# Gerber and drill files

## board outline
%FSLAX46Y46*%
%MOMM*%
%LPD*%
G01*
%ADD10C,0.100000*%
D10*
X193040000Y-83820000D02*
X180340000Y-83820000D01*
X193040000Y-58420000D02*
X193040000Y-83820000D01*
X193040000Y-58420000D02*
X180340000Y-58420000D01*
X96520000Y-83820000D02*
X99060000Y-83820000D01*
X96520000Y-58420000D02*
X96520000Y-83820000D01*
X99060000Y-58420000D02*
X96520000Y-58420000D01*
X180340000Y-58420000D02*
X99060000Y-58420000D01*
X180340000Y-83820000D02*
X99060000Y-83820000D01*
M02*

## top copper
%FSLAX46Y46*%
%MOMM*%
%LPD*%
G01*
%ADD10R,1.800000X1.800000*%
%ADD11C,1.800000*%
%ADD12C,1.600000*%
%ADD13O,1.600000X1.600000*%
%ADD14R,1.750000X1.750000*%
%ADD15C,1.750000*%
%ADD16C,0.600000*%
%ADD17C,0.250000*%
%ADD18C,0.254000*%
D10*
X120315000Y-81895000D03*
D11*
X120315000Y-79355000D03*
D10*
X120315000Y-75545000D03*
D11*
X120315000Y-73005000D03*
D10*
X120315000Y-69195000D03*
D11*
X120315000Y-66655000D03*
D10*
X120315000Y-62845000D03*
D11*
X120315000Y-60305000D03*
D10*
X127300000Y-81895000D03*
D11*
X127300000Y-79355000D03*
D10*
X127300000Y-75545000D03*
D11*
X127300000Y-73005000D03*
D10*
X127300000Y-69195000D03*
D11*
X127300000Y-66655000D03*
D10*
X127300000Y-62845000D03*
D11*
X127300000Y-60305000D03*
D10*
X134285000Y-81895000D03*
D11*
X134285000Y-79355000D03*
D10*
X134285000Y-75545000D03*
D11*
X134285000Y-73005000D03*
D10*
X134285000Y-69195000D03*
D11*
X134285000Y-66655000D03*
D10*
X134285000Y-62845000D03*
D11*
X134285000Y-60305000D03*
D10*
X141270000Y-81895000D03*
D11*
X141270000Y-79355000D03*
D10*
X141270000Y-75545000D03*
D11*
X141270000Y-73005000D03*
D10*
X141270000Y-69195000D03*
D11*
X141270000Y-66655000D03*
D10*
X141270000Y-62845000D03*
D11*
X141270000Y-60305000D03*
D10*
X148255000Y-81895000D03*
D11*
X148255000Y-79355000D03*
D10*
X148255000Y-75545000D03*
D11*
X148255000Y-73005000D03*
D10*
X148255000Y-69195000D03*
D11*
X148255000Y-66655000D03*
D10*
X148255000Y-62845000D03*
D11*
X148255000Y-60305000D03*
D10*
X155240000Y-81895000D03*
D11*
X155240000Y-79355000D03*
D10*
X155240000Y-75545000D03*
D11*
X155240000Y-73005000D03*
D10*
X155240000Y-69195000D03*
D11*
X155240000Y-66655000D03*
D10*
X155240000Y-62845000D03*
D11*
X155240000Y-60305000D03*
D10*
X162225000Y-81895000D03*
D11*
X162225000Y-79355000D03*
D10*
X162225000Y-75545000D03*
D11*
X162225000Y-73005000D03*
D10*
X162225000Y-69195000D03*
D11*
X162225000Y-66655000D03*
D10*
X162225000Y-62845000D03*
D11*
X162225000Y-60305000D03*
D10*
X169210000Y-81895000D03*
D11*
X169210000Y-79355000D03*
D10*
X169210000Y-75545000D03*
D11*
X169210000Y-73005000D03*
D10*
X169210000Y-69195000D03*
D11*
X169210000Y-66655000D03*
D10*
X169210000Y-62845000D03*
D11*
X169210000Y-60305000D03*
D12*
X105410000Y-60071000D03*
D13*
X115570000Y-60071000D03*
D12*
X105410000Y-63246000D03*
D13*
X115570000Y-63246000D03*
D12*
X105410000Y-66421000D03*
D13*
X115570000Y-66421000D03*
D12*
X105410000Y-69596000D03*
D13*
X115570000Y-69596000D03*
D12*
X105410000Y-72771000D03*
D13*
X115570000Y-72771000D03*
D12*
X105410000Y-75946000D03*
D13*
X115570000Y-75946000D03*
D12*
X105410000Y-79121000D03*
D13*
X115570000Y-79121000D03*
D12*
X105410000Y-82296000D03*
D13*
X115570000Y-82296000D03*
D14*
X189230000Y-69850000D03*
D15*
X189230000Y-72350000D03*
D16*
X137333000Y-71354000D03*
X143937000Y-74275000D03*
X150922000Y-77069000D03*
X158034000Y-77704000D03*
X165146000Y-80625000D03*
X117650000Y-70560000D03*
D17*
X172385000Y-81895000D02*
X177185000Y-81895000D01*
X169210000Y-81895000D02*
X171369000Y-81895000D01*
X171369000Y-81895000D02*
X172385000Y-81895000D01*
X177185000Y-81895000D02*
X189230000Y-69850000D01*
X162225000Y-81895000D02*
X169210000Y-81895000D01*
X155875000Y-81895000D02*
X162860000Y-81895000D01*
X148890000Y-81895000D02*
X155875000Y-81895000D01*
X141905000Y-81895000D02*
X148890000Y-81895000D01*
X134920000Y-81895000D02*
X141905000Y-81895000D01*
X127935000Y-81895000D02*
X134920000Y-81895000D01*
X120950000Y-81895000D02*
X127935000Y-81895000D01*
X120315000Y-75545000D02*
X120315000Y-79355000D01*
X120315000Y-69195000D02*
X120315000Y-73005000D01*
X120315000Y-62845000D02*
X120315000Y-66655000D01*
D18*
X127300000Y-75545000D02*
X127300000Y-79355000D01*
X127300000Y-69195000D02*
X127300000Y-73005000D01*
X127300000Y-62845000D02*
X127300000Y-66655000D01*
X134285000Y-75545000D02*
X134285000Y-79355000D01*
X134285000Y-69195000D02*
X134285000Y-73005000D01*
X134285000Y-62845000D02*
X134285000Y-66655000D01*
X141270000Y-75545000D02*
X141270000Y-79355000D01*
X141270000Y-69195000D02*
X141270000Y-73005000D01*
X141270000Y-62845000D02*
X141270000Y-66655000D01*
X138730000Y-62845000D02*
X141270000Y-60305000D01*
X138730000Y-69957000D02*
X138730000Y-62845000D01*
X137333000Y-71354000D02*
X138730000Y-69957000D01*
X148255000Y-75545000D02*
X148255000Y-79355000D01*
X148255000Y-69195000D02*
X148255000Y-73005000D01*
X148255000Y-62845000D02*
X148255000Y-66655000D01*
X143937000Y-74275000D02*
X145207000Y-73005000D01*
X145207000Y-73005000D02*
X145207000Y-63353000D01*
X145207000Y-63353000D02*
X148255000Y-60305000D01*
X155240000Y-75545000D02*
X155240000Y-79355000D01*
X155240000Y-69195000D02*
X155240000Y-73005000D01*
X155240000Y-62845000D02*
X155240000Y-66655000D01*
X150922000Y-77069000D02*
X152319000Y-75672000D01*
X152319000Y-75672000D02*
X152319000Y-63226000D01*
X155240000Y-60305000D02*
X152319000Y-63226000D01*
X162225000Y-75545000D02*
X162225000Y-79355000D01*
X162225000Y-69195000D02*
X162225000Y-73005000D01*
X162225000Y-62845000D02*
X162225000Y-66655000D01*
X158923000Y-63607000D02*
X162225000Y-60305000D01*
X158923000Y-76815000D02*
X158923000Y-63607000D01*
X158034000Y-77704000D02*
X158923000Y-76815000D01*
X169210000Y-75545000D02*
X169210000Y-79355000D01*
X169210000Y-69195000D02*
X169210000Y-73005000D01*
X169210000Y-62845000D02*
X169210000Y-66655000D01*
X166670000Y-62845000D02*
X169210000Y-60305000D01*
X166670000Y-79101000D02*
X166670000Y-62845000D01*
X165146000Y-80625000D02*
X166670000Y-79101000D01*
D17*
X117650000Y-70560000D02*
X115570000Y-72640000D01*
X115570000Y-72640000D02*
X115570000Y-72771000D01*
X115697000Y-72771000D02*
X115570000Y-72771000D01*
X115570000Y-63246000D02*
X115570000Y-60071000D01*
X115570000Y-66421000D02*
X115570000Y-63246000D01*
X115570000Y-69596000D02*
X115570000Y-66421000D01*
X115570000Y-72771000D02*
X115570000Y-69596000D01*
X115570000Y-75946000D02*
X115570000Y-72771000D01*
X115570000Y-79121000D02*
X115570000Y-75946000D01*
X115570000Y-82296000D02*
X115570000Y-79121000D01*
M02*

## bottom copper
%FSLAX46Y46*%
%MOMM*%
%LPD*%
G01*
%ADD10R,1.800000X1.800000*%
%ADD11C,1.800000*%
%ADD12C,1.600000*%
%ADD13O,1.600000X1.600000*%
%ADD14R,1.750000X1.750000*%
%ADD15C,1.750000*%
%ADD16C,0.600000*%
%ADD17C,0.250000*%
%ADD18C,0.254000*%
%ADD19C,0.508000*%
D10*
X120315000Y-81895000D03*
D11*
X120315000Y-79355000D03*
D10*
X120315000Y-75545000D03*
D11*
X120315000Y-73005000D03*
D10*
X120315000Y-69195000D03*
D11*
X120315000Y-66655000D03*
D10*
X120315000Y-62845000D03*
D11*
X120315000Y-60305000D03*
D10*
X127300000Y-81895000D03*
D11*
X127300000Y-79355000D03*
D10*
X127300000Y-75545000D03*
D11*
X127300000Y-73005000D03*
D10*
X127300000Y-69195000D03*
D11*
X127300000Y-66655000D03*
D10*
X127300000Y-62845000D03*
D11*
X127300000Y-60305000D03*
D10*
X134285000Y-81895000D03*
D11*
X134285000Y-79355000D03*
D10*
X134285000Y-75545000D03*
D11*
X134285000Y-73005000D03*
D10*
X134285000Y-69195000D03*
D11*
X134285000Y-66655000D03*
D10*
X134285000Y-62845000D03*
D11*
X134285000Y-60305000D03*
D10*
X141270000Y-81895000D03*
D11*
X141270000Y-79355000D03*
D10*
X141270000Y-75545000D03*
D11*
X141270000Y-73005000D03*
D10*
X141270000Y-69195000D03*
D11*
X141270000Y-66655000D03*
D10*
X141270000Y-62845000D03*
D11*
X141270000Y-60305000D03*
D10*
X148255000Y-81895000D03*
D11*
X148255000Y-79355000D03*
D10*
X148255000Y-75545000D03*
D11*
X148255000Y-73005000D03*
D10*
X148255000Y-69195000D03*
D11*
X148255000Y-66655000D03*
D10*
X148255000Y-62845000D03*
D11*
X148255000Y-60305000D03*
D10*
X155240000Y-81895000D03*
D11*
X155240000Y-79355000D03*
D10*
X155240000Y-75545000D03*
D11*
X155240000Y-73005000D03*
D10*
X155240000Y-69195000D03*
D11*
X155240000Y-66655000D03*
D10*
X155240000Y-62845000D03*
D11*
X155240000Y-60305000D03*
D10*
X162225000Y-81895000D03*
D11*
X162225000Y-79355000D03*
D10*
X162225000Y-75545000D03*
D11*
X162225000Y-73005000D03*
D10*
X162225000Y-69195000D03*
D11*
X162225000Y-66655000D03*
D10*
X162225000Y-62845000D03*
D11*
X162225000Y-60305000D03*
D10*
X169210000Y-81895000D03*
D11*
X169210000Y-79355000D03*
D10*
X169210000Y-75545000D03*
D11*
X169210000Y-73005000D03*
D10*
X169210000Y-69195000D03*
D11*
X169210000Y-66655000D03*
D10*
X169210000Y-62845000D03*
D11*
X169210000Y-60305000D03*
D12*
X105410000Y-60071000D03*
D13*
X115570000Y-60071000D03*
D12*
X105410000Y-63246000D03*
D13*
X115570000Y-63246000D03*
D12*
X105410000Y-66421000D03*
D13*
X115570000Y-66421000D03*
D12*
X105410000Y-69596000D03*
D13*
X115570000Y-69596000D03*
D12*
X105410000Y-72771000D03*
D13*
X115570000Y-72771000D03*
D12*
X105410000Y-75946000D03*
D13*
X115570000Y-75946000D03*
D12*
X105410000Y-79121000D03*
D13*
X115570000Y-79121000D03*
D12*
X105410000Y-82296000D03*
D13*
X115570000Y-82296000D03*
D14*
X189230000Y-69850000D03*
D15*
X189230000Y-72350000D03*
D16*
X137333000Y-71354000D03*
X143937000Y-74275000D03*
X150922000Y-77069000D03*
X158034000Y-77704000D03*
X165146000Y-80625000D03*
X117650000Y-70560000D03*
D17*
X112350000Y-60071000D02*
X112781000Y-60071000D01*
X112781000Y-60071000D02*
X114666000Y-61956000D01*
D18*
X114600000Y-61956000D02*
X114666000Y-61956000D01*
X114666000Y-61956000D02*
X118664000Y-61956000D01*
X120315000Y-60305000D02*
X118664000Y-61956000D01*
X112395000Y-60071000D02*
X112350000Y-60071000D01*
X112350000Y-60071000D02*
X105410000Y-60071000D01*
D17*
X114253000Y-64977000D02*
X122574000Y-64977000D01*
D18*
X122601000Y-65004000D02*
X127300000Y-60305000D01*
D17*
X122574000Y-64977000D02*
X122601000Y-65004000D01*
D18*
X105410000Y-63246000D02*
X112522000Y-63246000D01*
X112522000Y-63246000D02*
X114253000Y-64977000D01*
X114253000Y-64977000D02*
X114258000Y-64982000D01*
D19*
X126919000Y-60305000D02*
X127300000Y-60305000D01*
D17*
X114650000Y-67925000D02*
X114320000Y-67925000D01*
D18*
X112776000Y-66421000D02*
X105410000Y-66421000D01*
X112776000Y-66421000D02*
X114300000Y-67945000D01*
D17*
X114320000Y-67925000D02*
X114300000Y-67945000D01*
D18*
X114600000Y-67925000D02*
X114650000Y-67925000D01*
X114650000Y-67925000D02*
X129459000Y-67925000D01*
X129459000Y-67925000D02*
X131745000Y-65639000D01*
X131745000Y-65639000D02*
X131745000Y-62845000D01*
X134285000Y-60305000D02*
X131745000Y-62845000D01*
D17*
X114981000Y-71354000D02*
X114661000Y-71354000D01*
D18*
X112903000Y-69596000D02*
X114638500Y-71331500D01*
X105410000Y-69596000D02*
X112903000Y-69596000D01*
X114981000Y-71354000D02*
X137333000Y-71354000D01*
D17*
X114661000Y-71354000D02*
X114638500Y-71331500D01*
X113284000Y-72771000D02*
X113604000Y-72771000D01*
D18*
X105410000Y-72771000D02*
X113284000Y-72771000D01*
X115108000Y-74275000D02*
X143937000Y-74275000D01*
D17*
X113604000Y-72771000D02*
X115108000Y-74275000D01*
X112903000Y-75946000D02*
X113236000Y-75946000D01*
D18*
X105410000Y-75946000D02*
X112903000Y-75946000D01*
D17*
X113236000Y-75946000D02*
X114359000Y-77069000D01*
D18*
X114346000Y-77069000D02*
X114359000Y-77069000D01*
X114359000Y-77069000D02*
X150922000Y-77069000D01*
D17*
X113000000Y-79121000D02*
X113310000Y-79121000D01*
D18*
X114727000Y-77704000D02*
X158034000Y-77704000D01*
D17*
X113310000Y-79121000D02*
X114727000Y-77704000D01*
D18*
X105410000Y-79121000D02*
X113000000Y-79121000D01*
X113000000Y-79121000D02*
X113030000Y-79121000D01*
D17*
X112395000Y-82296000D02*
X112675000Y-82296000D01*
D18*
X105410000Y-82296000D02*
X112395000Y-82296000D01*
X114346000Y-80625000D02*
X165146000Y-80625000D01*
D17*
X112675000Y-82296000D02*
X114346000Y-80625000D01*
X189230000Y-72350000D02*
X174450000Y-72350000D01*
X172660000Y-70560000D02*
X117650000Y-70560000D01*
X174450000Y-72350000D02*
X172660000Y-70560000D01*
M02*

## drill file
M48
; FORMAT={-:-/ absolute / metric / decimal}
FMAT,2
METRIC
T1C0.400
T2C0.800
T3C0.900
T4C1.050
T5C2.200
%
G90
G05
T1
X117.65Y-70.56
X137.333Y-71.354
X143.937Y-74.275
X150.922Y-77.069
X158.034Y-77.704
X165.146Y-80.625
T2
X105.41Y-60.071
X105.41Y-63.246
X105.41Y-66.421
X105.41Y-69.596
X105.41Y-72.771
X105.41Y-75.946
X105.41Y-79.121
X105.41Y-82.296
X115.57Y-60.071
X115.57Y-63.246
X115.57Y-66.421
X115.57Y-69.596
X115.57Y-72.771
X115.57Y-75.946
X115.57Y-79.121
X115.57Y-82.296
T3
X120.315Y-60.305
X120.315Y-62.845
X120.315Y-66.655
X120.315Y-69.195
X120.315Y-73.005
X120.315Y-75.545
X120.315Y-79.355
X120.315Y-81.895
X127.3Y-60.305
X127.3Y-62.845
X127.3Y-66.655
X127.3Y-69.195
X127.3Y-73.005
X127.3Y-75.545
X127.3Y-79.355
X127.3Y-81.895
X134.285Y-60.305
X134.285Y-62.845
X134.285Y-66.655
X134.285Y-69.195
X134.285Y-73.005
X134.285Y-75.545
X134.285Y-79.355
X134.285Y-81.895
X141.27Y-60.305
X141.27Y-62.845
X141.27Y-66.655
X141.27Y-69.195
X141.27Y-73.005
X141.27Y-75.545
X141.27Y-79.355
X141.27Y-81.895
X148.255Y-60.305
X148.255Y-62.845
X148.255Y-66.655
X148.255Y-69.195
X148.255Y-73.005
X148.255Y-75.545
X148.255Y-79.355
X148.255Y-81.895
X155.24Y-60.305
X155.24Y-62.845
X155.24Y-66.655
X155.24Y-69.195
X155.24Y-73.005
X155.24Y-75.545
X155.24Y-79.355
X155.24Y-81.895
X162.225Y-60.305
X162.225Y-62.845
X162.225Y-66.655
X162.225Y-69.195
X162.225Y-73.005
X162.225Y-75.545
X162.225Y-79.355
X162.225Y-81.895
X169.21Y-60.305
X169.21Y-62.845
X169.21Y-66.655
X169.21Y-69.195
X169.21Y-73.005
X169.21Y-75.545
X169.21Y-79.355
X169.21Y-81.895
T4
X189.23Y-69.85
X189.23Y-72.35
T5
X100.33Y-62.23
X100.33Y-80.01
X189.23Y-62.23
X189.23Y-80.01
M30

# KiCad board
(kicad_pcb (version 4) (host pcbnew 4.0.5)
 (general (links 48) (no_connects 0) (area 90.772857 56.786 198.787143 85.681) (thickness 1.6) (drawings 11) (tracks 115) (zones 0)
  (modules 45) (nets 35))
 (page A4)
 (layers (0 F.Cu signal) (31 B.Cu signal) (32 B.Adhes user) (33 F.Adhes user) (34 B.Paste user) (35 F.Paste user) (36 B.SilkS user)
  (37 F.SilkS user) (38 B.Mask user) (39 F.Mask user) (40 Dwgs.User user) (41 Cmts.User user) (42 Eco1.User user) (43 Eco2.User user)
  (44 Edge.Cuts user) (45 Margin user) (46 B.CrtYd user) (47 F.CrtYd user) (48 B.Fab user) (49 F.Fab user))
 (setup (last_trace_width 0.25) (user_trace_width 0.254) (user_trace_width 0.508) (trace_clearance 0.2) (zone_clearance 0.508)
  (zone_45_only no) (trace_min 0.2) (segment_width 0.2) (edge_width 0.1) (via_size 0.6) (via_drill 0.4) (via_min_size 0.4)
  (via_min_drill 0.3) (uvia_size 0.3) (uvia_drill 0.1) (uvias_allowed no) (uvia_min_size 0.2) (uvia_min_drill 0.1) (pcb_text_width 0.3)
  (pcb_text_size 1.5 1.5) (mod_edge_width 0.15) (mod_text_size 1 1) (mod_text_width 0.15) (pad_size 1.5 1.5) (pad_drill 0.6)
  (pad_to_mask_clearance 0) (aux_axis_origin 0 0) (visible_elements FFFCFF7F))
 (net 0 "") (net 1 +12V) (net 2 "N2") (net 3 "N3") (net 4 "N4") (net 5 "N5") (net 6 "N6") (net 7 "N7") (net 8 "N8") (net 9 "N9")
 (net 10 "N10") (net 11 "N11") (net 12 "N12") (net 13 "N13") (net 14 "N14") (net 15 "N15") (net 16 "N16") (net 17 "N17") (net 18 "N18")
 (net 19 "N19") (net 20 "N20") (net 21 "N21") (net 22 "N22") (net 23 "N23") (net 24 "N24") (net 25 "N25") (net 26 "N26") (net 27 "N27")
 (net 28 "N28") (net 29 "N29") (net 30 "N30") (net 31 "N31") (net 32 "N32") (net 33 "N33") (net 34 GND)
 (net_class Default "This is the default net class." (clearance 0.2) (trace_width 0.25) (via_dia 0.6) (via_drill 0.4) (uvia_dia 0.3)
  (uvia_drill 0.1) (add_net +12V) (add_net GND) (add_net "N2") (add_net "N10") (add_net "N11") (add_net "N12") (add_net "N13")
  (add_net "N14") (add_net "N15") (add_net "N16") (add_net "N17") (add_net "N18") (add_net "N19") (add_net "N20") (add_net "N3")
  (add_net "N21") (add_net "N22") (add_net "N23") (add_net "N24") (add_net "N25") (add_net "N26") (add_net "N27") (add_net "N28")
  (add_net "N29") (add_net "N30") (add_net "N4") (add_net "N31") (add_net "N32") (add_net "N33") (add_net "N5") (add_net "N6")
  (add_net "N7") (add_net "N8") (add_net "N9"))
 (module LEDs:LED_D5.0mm (layer F.Cu) (at 120.315 81.895 90)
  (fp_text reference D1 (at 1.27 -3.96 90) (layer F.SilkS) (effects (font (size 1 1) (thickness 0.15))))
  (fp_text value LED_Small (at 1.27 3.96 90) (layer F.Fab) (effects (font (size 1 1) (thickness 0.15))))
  (pad 1 thru_hole rect (at 0 0 90) (size 1.8 1.8) (drill 0.9) (layers *.Cu *.Mask) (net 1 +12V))
  (pad 2 thru_hole circle (at 2.54 0 90) (size 1.8 1.8) (drill 0.9) (layers *.Cu *.Mask) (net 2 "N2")))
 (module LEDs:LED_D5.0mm (layer F.Cu) (at 120.315 75.545 90)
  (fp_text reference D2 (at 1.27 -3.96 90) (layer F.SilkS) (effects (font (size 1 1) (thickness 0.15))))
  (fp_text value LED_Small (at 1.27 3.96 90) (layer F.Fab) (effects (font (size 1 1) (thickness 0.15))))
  (pad 1 thru_hole rect (at 0 0 90) (size 1.8 1.8) (drill 0.9) (layers *.Cu *.Mask) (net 2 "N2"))
  (pad 2 thru_hole circle (at 2.54 0 90) (size 1.8 1.8) (drill 0.9) (layers *.Cu *.Mask) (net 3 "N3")))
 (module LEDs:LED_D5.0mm (layer F.Cu) (at 120.315 69.195 90)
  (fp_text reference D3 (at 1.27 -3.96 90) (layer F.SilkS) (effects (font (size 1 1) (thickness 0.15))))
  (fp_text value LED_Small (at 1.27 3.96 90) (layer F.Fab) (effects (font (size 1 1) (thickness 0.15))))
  (pad 1 thru_hole rect (at 0 0 90) (size 1.8 1.8) (drill 0.9) (layers *.Cu *.Mask) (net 3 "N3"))
  (pad 2 thru_hole circle (at 2.54 0 90) (size 1.8 1.8) (drill 0.9) (layers *.Cu *.Mask) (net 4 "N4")))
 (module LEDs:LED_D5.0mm (layer F.Cu) (at 120.315 62.845 90)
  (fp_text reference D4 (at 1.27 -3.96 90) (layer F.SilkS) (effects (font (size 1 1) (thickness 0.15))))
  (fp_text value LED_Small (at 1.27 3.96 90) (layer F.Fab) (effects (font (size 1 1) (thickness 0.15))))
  (pad 1 thru_hole rect (at 0 0 90) (size 1.8 1.8) (drill 0.9) (layers *.Cu *.Mask) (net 4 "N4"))
  (pad 2 thru_hole circle (at 2.54 0 90) (size 1.8 1.8) (drill 0.9) (layers *.Cu *.Mask) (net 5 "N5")))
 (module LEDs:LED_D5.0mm (layer F.Cu) (at 127.3 81.895 90)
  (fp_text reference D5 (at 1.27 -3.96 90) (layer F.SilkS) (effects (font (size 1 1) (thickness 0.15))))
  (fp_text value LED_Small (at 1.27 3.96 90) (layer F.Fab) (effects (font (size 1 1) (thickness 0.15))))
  (pad 1 thru_hole rect (at 0 0 90) (size 1.8 1.8) (drill 0.9) (layers *.Cu *.Mask) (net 1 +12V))
  (pad 2 thru_hole circle (at 2.54 0 90) (size 1.8 1.8) (drill 0.9) (layers *.Cu *.Mask) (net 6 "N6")))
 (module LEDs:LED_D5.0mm (layer F.Cu) (at 127.3 75.545 90)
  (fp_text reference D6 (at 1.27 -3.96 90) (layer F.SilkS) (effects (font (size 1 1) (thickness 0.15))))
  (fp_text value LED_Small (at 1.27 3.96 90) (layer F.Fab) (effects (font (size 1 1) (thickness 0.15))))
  (pad 1 thru_hole rect (at 0 0 90) (size 1.8 1.8) (drill 0.9) (layers *.Cu *.Mask) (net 6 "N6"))
  (pad 2 thru_hole circle (at 2.54 0 90) (size 1.8 1.8) (drill 0.9) (layers *.Cu *.Mask) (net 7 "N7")))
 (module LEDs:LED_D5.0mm (layer F.Cu) (at 127.3 69.195 90)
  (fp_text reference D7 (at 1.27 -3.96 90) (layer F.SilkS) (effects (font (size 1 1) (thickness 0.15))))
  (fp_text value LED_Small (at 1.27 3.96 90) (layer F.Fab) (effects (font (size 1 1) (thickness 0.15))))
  (pad 1 thru_hole rect (at 0 0 90) (size 1.8 1.8) (drill 0.9) (layers *.Cu *.Mask) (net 7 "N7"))
  (pad 2 thru_hole circle (at 2.54 0 90) (size 1.8 1.8) (drill 0.9) (layers *.Cu *.Mask) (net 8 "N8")))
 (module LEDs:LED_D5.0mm (layer F.Cu) (at 127.3 62.845 90)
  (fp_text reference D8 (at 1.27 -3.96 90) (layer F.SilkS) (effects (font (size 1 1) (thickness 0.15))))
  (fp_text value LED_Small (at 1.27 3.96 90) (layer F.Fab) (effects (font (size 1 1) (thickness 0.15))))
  (pad 1 thru_hole rect (at 0 0 90) (size 1.8 1.8) (drill 0.9) (layers *.Cu *.Mask) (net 8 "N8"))
  (pad 2 thru_hole circle (at 2.54 0 90) (size 1.8 1.8) (drill 0.9) (layers *.Cu *.Mask) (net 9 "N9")))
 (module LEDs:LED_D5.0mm (layer F.Cu) (at 134.285 81.895 90)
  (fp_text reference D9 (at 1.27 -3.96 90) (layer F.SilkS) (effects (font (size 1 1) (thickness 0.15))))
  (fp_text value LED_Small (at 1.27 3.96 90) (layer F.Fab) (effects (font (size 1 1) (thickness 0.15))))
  (pad 1 thru_hole rect (at 0 0 90) (size 1.8 1.8) (drill 0.9) (layers *.Cu *.Mask) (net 1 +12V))
  (pad 2 thru_hole circle (at 2.54 0 90) (size 1.8 1.8) (drill 0.9) (layers *.Cu *.Mask) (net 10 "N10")))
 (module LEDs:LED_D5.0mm (layer F.Cu) (at 134.285 75.545 90)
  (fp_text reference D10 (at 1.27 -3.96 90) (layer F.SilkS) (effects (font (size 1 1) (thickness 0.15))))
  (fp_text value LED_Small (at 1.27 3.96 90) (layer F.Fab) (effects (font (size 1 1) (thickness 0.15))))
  (pad 1 thru_hole rect (at 0 0 90) (size 1.8 1.8) (drill 0.9) (layers *.Cu *.Mask) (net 10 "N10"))
  (pad 2 thru_hole circle (at 2.54 0 90) (size 1.8 1.8) (drill 0.9) (layers *.Cu *.Mask) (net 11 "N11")))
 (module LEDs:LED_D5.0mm (layer F.Cu) (at 134.285 69.195 90)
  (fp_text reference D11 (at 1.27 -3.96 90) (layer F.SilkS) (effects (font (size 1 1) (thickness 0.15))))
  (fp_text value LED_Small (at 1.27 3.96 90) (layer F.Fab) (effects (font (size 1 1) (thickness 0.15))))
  (pad 1 thru_hole rect (at 0 0 90) (size 1.8 1.8) (drill 0.9) (layers *.Cu *.Mask) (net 11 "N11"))
  (pad 2 thru_hole circle (at 2.54 0 90) (size 1.8 1.8) (drill 0.9) (layers *.Cu *.Mask) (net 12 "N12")))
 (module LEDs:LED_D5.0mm (layer F.Cu) (at 134.285 62.845 90)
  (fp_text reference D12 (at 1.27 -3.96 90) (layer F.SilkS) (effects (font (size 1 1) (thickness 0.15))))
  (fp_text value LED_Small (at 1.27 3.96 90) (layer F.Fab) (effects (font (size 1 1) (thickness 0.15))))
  (pad 1 thru_hole rect (at 0 0 90) (size 1.8 1.8) (drill 0.9) (layers *.Cu *.Mask) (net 12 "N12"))
  (pad 2 thru_hole circle (at 2.54 0 90) (size 1.8 1.8) (drill 0.9) (layers *.Cu *.Mask) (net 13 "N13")))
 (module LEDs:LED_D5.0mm (layer F.Cu) (at 141.27 81.895 90)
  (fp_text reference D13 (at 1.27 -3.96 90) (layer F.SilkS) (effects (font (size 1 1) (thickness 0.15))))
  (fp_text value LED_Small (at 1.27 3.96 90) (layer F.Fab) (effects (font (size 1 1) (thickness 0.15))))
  (pad 1 thru_hole rect (at 0 0 90) (size 1.8 1.8) (drill 0.9) (layers *.Cu *.Mask) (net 1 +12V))
  (pad 2 thru_hole circle (at 2.54 0 90) (size 1.8 1.8) (drill 0.9) (layers *.Cu *.Mask) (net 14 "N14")))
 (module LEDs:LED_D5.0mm (layer F.Cu) (at 141.27 75.545 90)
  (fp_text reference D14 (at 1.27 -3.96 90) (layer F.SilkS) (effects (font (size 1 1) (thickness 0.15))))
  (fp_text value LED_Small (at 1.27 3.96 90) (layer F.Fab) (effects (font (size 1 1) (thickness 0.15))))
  (pad 1 thru_hole rect (at 0 0 90) (size 1.8 1.8) (drill 0.9) (layers *.Cu *.Mask) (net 14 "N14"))
  (pad 2 thru_hole circle (at 2.54 0 90) (size 1.8 1.8) (drill 0.9) (layers *.Cu *.Mask) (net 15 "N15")))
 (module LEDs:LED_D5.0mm (layer F.Cu) (at 141.27 69.195 90)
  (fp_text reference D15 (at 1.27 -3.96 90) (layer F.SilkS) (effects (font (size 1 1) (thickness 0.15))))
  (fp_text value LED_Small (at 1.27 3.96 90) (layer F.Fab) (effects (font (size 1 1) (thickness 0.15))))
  (pad 1 thru_hole rect (at 0 0 90) (size 1.8 1.8) (drill 0.9) (layers *.Cu *.Mask) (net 15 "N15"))
  (pad 2 thru_hole circle (at 2.54 0 90) (size 1.8 1.8) (drill 0.9) (layers *.Cu *.Mask) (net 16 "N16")))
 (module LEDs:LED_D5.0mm (layer F.Cu) (at 141.27 62.845 90)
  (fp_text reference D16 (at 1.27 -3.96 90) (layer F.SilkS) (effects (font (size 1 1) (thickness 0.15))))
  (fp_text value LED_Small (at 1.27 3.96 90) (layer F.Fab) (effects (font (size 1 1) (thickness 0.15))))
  (pad 1 thru_hole rect (at 0 0 90) (size 1.8 1.8) (drill 0.9) (layers *.Cu *.Mask) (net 16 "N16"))
  (pad 2 thru_hole circle (at 2.54 0 90) (size 1.8 1.8) (drill 0.9) (layers *.Cu *.Mask) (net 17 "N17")))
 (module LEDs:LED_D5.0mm (layer F.Cu) (at 148.255 81.895 90)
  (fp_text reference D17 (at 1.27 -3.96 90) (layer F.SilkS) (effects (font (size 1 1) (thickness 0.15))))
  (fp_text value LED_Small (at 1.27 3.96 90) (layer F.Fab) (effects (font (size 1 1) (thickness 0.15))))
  (pad 1 thru_hole rect (at 0 0 90) (size 1.8 1.8) (drill 0.9) (layers *.Cu *.Mask) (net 1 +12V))
  (pad 2 thru_hole circle (at 2.54 0 90) (size 1.8 1.8) (drill 0.9) (layers *.Cu *.Mask) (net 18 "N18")))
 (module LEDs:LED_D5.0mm (layer F.Cu) (at 148.255 75.545 90)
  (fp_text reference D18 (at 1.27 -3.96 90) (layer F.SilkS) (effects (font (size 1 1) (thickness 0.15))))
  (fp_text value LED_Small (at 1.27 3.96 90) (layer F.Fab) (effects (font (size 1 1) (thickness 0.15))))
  (pad 1 thru_hole rect (at 0 0 90) (size 1.8 1.8) (drill 0.9) (layers *.Cu *.Mask) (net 18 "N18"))
  (pad 2 thru_hole circle (at 2.54 0 90) (size 1.8 1.8) (drill 0.9) (layers *.Cu *.Mask) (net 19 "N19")))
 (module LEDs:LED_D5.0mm (layer F.Cu) (at 148.255 69.195 90)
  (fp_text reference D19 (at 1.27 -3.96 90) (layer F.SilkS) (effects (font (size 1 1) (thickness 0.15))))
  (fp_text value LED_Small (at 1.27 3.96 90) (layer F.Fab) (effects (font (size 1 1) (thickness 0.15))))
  (pad 1 thru_hole rect (at 0 0 90) (size 1.8 1.8) (drill 0.9) (layers *.Cu *.Mask) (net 19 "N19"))
  (pad 2 thru_hole circle (at 2.54 0 90) (size 1.8 1.8) (drill 0.9) (layers *.Cu *.Mask) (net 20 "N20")))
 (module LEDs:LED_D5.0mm (layer F.Cu) (at 148.255 62.845 90)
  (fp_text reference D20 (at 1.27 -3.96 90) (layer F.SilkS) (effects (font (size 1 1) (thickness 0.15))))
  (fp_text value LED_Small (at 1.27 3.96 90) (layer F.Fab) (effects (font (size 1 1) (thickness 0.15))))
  (pad 1 thru_hole rect (at 0 0 90) (size 1.8 1.8) (drill 0.9) (layers *.Cu *.Mask) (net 20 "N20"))
  (pad 2 thru_hole circle (at 2.54 0 90) (size 1.8 1.8) (drill 0.9) (layers *.Cu *.Mask) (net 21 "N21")))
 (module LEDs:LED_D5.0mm (layer F.Cu) (at 155.24 81.895 90)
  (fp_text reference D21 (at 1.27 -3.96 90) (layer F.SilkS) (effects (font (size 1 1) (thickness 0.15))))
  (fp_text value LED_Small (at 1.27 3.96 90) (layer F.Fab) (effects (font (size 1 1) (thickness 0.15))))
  (pad 1 thru_hole rect (at 0 0 90) (size 1.8 1.8) (drill 0.9) (layers *.Cu *.Mask) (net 1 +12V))
  (pad 2 thru_hole circle (at 2.54 0 90) (size 1.8 1.8) (drill 0.9) (layers *.Cu *.Mask) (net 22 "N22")))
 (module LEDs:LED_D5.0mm (layer F.Cu) (at 155.24 75.545 90)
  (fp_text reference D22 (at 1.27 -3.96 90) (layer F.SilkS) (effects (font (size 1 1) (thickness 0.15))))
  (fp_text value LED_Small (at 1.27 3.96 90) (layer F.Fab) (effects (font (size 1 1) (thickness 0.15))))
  (pad 1 thru_hole rect (at 0 0 90) (size 1.8 1.8) (drill 0.9) (layers *.Cu *.Mask) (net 22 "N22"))
  (pad 2 thru_hole circle (at 2.54 0 90) (size 1.8 1.8) (drill 0.9) (layers *.Cu *.Mask) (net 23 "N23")))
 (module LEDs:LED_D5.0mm (layer F.Cu) (at 155.24 69.195 90)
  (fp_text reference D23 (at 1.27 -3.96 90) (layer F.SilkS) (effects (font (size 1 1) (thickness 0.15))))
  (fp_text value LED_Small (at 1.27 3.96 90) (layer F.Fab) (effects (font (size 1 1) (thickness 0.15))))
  (pad 1 thru_hole rect (at 0 0 90) (size 1.8 1.8) (drill 0.9) (layers *.Cu *.Mask) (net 23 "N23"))
  (pad 2 thru_hole circle (at 2.54 0 90) (size 1.8 1.8) (drill 0.9) (layers *.Cu *.Mask) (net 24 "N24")))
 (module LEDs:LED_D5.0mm (layer F.Cu) (at 155.24 62.845 90)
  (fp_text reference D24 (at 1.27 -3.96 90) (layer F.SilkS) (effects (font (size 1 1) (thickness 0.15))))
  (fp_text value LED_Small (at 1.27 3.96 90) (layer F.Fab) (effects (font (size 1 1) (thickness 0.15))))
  (pad 1 thru_hole rect (at 0 0 90) (size 1.8 1.8) (drill 0.9) (layers *.Cu *.Mask) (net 24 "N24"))
  (pad 2 thru_hole circle (at 2.54 0 90) (size 1.8 1.8) (drill 0.9) (layers *.Cu *.Mask) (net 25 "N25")))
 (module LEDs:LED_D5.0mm (layer F.Cu) (at 162.225 81.895 90)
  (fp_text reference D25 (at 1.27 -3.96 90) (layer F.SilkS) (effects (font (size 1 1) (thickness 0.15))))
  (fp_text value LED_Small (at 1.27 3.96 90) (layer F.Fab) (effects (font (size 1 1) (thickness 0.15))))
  (pad 1 thru_hole rect (at 0 0 90) (size 1.8 1.8) (drill 0.9) (layers *.Cu *.Mask) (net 1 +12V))
  (pad 2 thru_hole circle (at 2.54 0 90) (size 1.8 1.8) (drill 0.9) (layers *.Cu *.Mask) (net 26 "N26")))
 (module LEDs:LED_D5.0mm (layer F.Cu) (at 162.225 75.545 90)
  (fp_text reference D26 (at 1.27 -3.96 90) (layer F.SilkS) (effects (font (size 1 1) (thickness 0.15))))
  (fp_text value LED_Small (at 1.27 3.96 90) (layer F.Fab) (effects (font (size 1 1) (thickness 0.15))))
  (pad 1 thru_hole rect (at 0 0 90) (size 1.8 1.8) (drill 0.9) (layers *.Cu *.Mask) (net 26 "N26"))
  (pad 2 thru_hole circle (at 2.54 0 90) (size 1.8 1.8) (drill 0.9) (layers *.Cu *.Mask) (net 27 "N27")))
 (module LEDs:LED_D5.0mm (layer F.Cu) (at 162.225 69.195 90)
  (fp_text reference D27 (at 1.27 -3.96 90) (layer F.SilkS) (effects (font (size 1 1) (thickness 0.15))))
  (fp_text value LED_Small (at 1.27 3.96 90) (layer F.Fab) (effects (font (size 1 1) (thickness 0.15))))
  (pad 1 thru_hole rect (at 0 0 90) (size 1.8 1.8) (drill 0.9) (layers *.Cu *.Mask) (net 27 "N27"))
  (pad 2 thru_hole circle (at 2.54 0 90) (size 1.8 1.8) (drill 0.9) (layers *.Cu *.Mask) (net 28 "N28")))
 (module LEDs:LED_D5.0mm (layer F.Cu) (at 162.225 62.845 90)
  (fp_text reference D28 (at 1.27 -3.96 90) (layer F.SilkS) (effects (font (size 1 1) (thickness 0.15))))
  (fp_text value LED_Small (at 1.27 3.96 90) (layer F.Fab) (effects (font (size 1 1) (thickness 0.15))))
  (pad 1 thru_hole rect (at 0 0 90) (size 1.8 1.8) (drill 0.9) (layers *.Cu *.Mask) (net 28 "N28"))
  (pad 2 thru_hole circle (at 2.54 0 90) (size 1.8 1.8) (drill 0.9) (layers *.Cu *.Mask) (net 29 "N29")))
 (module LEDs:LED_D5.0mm (layer F.Cu) (at 169.21 81.895 90)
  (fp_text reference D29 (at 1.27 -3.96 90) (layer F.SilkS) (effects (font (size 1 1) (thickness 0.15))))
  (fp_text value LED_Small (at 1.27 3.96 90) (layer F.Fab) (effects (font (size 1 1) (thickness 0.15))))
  (pad 1 thru_hole rect (at 0 0 90) (size 1.8 1.8) (drill 0.9) (layers *.Cu *.Mask) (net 1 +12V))
  (pad 2 thru_hole circle (at 2.54 0 90) (size 1.8 1.8) (drill 0.9) (layers *.Cu *.Mask) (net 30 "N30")))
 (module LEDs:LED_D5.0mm (layer F.Cu) (at 169.21 75.545 90)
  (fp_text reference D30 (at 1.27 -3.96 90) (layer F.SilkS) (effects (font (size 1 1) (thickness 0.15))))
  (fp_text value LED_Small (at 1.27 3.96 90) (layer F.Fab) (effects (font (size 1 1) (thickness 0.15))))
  (pad 1 thru_hole rect (at 0 0 90) (size 1.8 1.8) (drill 0.9) (layers *.Cu *.Mask) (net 30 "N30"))
  (pad 2 thru_hole circle (at 2.54 0 90) (size 1.8 1.8) (drill 0.9) (layers *.Cu *.Mask) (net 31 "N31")))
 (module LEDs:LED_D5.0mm (layer F.Cu) (at 169.21 69.195 90)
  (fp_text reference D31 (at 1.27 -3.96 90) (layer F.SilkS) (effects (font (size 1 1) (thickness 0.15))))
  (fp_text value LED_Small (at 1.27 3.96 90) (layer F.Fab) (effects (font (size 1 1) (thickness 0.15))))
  (pad 1 thru_hole rect (at 0 0 90) (size 1.8 1.8) (drill 0.9) (layers *.Cu *.Mask) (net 31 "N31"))
  (pad 2 thru_hole circle (at 2.54 0 90) (size 1.8 1.8) (drill 0.9) (layers *.Cu *.Mask) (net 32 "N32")))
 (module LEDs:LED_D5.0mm (layer F.Cu) (at 169.21 62.845 90)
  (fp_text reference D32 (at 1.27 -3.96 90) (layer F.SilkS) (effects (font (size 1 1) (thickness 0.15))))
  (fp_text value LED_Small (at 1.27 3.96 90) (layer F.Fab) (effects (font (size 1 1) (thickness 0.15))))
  (pad 1 thru_hole rect (at 0 0 90) (size 1.8 1.8) (drill 0.9) (layers *.Cu *.Mask) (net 32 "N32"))
  (pad 2 thru_hole circle (at 2.54 0 90) (size 1.8 1.8) (drill 0.9) (layers *.Cu *.Mask) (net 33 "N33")))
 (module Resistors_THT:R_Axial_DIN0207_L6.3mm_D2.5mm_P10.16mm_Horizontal (layer F.Cu) (at 105.41 60.071)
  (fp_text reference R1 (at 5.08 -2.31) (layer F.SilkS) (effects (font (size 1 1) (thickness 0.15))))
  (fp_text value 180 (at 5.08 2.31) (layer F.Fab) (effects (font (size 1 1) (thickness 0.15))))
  (pad 1 thru_hole circle (at 0 0) (size 1.6 1.6) (drill 0.8) (layers *.Cu *.Mask) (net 5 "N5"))
  (pad 2 thru_hole oval (at 10.16 0) (size 1.6 1.6) (drill 0.8) (layers *.Cu *.Mask) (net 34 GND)))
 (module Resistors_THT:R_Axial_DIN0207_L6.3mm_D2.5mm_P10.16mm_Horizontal (layer F.Cu) (at 105.41 63.246)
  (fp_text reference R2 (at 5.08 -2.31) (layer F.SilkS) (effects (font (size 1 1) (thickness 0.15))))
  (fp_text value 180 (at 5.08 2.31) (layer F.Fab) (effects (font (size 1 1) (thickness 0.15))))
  (pad 1 thru_hole circle (at 0 0) (size 1.6 1.6) (drill 0.8) (layers *.Cu *.Mask) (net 9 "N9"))
  (pad 2 thru_hole oval (at 10.16 0) (size 1.6 1.6) (drill 0.8) (layers *.Cu *.Mask) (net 34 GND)))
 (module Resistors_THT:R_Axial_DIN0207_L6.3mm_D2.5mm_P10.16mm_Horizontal (layer F.Cu) (at 105.41 66.421)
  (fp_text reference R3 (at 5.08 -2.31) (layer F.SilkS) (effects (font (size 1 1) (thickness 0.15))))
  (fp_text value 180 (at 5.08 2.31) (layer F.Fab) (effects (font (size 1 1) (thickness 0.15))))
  (pad 1 thru_hole circle (at 0 0) (size 1.6 1.6) (drill 0.8) (layers *.Cu *.Mask) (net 13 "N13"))
  (pad 2 thru_hole oval (at 10.16 0) (size 1.6 1.6) (drill 0.8) (layers *.Cu *.Mask) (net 34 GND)))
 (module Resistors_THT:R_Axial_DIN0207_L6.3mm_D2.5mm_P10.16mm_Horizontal (layer F.Cu) (at 105.41 69.596)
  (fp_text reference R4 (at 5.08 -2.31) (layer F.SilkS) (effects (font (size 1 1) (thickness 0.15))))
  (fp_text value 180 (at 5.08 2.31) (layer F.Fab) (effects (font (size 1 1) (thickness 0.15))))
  (pad 1 thru_hole circle (at 0 0) (size 1.6 1.6) (drill 0.8) (layers *.Cu *.Mask) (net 17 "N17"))
  (pad 2 thru_hole oval (at 10.16 0) (size 1.6 1.6) (drill 0.8) (layers *.Cu *.Mask) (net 34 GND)))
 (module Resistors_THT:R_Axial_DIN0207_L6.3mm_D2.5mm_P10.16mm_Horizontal (layer F.Cu) (at 105.41 72.771)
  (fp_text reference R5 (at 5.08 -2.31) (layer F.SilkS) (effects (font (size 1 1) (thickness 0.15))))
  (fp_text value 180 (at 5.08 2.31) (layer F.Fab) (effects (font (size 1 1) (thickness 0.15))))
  (pad 1 thru_hole circle (at 0 0) (size 1.6 1.6) (drill 0.8) (layers *.Cu *.Mask) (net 21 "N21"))
  (pad 2 thru_hole oval (at 10.16 0) (size 1.6 1.6) (drill 0.8) (layers *.Cu *.Mask) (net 34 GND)))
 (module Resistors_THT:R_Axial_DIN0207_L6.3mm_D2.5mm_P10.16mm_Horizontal (layer F.Cu) (at 105.41 75.946)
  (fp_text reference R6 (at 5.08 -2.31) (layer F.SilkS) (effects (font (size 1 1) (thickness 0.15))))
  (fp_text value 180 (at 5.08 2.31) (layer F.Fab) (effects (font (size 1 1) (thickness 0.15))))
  (pad 1 thru_hole circle (at 0 0) (size 1.6 1.6) (drill 0.8) (layers *.Cu *.Mask) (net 25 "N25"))
  (pad 2 thru_hole oval (at 10.16 0) (size 1.6 1.6) (drill 0.8) (layers *.Cu *.Mask) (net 34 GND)))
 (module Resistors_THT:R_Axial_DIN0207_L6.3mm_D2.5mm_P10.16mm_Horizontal (layer F.Cu) (at 105.41 79.121)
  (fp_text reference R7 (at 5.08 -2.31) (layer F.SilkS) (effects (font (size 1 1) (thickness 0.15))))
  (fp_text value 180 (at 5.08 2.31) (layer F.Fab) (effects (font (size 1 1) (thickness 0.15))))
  (pad 1 thru_hole circle (at 0 0) (size 1.6 1.6) (drill 0.8) (layers *.Cu *.Mask) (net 29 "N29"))
  (pad 2 thru_hole oval (at 10.16 0) (size 1.6 1.6) (drill 0.8) (layers *.Cu *.Mask) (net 34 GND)))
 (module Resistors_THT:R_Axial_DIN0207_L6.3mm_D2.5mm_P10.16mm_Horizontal (layer F.Cu) (at 105.41 82.296)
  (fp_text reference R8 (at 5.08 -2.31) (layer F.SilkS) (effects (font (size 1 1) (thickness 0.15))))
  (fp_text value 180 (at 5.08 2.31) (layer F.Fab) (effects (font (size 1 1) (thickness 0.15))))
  (pad 1 thru_hole circle (at 0 0) (size 1.6 1.6) (drill 0.8) (layers *.Cu *.Mask) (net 33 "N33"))
  (pad 2 thru_hole oval (at 10.16 0) (size 1.6 1.6) (drill 0.8) (layers *.Cu *.Mask) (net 34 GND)))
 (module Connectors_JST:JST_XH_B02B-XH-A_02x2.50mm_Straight (layer F.Cu) (at 189.23 69.85 270)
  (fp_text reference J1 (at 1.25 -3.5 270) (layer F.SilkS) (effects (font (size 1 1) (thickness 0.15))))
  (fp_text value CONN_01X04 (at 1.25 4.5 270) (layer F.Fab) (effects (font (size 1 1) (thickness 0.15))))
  (pad 1 thru_hole rect (at 0 0 270) (size 1.75 1.75) (drill 1.05) (layers *.Cu *.Mask) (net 1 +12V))
  (pad 2 thru_hole circle (at 2.5 0 270) (size 1.75 1.75) (drill 1.05) (layers *.Cu *.Mask) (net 34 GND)))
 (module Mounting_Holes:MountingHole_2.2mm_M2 (layer F.Cu) (at 189.23 62.23)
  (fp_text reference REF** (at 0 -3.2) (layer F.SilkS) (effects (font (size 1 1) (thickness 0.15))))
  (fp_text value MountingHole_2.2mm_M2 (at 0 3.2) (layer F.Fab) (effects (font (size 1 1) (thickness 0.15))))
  (pad 1 np_thru_hole circle (at 0 0) (size 2.2 2.2) (drill 2.2) (layers *.Cu *.Mask)))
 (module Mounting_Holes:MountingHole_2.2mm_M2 (layer F.Cu) (at 189.23 80.01)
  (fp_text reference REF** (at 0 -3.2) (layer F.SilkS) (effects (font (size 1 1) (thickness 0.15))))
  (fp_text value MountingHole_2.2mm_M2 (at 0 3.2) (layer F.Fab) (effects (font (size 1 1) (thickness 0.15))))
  (pad 1 np_thru_hole circle (at 0 0) (size 2.2 2.2) (drill 2.2) (layers *.Cu *.Mask)))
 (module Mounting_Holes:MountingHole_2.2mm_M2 (layer F.Cu) (at 100.33 62.23)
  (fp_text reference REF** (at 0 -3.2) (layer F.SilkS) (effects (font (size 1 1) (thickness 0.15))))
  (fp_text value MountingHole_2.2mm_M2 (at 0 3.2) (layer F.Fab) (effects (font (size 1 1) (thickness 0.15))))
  (pad 1 np_thru_hole circle (at 0 0) (size 2.2 2.2) (drill 2.2) (layers *.Cu *.Mask)))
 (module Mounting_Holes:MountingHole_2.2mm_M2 (layer F.Cu) (at 100.33 80.01)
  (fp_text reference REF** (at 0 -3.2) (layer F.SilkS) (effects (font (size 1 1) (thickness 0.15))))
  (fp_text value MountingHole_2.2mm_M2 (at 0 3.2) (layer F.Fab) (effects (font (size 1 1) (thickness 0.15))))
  (pad 1 np_thru_hole circle (at 0 0) (size 2.2 2.2) (drill 2.2) (layers *.Cu *.Mask)))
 (gr_line (start 193.04 83.82) (end 180.34 83.82) (angle 90) (layer Edge.Cuts) (width 0.1))
 (gr_line (start 193.04 58.42) (end 193.04 83.82) (angle 90) (layer Edge.Cuts) (width 0.1))
 (gr_line (start 193.04 58.42) (end 180.34 58.42) (angle 90) (layer Edge.Cuts) (width 0.1))
 (gr_line (start 96.52 83.82) (end 99.06 83.82) (angle 90) (layer Edge.Cuts) (width 0.1))
 (gr_line (start 96.52 58.42) (end 96.52 83.82) (angle 90) (layer Edge.Cuts) (width 0.1))
 (gr_line (start 99.06 58.42) (end 96.52 58.42) (angle 90) (layer Edge.Cuts) (width 0.1))
 (gr_line (start 180.34 58.42) (end 99.06 58.42) (angle 90) (layer Edge.Cuts) (width 0.1))
 (gr_line (start 180.34 83.82) (end 99.06 83.82) (angle 90) (layer Edge.Cuts) (width 0.1))
 (segment (start 172.385 81.895) (end 177.185 81.895) (width 0.25) (layer F.Cu) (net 1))
 (segment (start 169.21 81.895) (end 171.369 81.895) (width 0.25) (layer F.Cu) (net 1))
 (segment (start 171.369 81.895) (end 172.385 81.895) (width 0.25) (layer F.Cu) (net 1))
 (segment (start 177.185 81.895) (end 189.23 69.85) (width 0.25) (layer F.Cu) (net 1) (status 800000))
 (segment (start 162.225 81.895) (end 169.21 81.895) (width 0.25) (layer F.Cu) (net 1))
 (segment (start 155.875 81.895) (end 162.86 81.895) (width 0.25) (layer F.Cu) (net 1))
 (segment (start 148.89 81.895) (end 155.875 81.895) (width 0.25) (layer F.Cu) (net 1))
 (segment (start 141.905 81.895) (end 148.89 81.895) (width 0.25) (layer F.Cu) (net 1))
 (segment (start 134.92 81.895) (end 141.905 81.895) (width 0.25) (layer F.Cu) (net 1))
 (segment (start 127.935 81.895) (end 134.92 81.895) (width 0.25) (layer F.Cu) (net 1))
 (segment (start 120.95 81.895) (end 127.935 81.895) (width 0.25) (layer F.Cu) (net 1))
 (segment (start 120.315 75.545) (end 120.315 79.355) (width 0.25) (layer F.Cu) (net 2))
 (segment (start 120.315 69.195) (end 120.315 73.005) (width 0.25) (layer F.Cu) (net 3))
 (segment (start 120.315 62.845) (end 120.315 66.655) (width 0.25) (layer F.Cu) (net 4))
 (segment (start 112.35 60.071) (end 112.781 60.071) (width 0.25) (layer B.Cu) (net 5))
 (segment (start 112.781 60.071) (end 114.666 61.956) (width 0.25) (layer B.Cu) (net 5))
 (segment (start 114.6 61.956) (end 114.666 61.956) (width 0.254) (layer B.Cu) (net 5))
 (segment (start 114.666 61.956) (end 118.664 61.956) (width 0.254) (layer B.Cu) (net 5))
 (segment (start 120.315 60.305) (end 118.664 61.956) (width 0.254) (layer B.Cu) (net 5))
 (segment (start 112.395 60.071) (end 112.35 60.071) (width 0.254) (layer B.Cu) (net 5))
 (segment (start 112.35 60.071) (end 105.41 60.071) (width 0.254) (layer B.Cu) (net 5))
 (segment (start 127.3 75.545) (end 127.3 79.355) (width 0.254) (layer F.Cu) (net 6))
 (segment (start 127.3 69.195) (end 127.3 73.005) (width 0.254) (layer F.Cu) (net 7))
 (segment (start 127.3 62.845) (end 127.3 66.655) (width 0.254) (layer F.Cu) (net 8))
 (segment (start 114.253 64.977) (end 122.574 64.977) (width 0.25) (layer B.Cu) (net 9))
 (segment (start 122.601 65.004) (end 127.3 60.305) (width 0.254) (layer B.Cu) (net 9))
 (segment (start 122.574 64.977) (end 122.601 65.004) (width 0.25) (layer B.Cu) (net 9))
 (segment (start 105.41 63.246) (end 112.522 63.246) (width 0.254) (layer B.Cu) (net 9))
 (segment (start 112.522 63.246) (end 114.253 64.977) (width 0.254) (layer B.Cu) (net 9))
 (segment (start 114.253 64.977) (end 114.258 64.982) (width 0.254) (layer B.Cu) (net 9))
 (segment (start 126.919 60.305) (end 127.3 60.305) (width 0.508) (layer B.Cu) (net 9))
 (segment (start 134.285 75.545) (end 134.285 79.355) (width 0.254) (layer F.Cu) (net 10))
 (segment (start 134.285 69.195) (end 134.285 73.005) (width 0.254) (layer F.Cu) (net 11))
 (segment (start 134.285 62.845) (end 134.285 66.655) (width 0.254) (layer F.Cu) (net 12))
 (segment (start 114.65 67.925) (end 114.32 67.925) (width 0.25) (layer B.Cu) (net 13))
 (segment (start 112.776 66.421) (end 105.41 66.421) (width 0.254) (layer B.Cu) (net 13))
 (segment (start 112.776 66.421) (end 114.3 67.945) (width 0.254) (layer B.Cu) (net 13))
 (segment (start 114.32 67.925) (end 114.3 67.945) (width 0.25) (layer B.Cu) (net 13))
 (segment (start 114.6 67.925) (end 114.65 67.925) (width 0.254) (layer B.Cu) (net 13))
 (segment (start 114.65 67.925) (end 129.459 67.925) (width 0.254) (layer B.Cu) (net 13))
 (segment (start 129.459 67.925) (end 131.745 65.639) (width 0.254) (layer B.Cu) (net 13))
 (segment (start 131.745 65.639) (end 131.745 62.845) (width 0.254) (layer B.Cu) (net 13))
 (segment (start 134.285 60.305) (end 131.745 62.845) (width 0.254) (layer B.Cu) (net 13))
 (segment (start 141.27 75.545) (end 141.27 79.355) (width 0.254) (layer F.Cu) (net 14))
 (segment (start 141.27 69.195) (end 141.27 73.005) (width 0.254) (layer F.Cu) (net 15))
 (segment (start 141.27 62.845) (end 141.27 66.655) (width 0.254) (layer F.Cu) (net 16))
 (segment (start 114.981 71.354) (end 114.661 71.354) (width 0.25) (layer B.Cu) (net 17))
 (segment (start 112.903 69.596) (end 114.6385 71.3315) (width 0.254) (layer B.Cu) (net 17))
 (segment (start 105.41 69.596) (end 112.903 69.596) (width 0.254) (layer B.Cu) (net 17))
 (segment (start 138.73 62.845) (end 141.27 60.305) (width 0.254) (layer F.Cu) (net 17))
 (segment (start 138.73 69.957) (end 138.73 62.845) (width 0.254) (layer F.Cu) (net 17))
 (segment (start 137.333 71.354) (end 138.73 69.957) (width 0.254) (layer F.Cu) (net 17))
 (via (at 137.333 71.354) (size 0.6) (drill 0.4) (layers F.Cu B.Cu) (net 17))
 (segment (start 114.981 71.354) (end 137.333 71.354) (width 0.254) (layer B.Cu) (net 17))
 (segment (start 114.661 71.354) (end 114.6385 71.3315) (width 0.25) (layer B.Cu) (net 17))
 (segment (start 148.255 75.545) (end 148.255 79.355) (width 0.254) (layer F.Cu) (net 18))
 (segment (start 148.255 69.195) (end 148.255 73.005) (width 0.254) (layer F.Cu) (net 19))
 (segment (start 148.255 62.845) (end 148.255 66.655) (width 0.254) (layer F.Cu) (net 20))
 (segment (start 113.284 72.771) (end 113.604 72.771) (width 0.25) (layer B.Cu) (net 21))
 (segment (start 105.41 72.771) (end 113.284 72.771) (width 0.254) (layer B.Cu) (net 21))
 (segment (start 115.108 74.275) (end 143.937 74.275) (width 0.254) (layer B.Cu) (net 21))
 (via (at 143.937 74.275) (size 0.6) (drill 0.4) (layers F.Cu B.Cu) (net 21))
 (segment (start 143.937 74.275) (end 145.207 73.005) (width 0.254) (layer F.Cu) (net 21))
 (segment (start 145.207 73.005) (end 145.207 63.353) (width 0.254) (layer F.Cu) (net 21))
 (segment (start 145.207 63.353) (end 148.255 60.305) (width 0.254) (layer F.Cu) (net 21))
 (segment (start 113.604 72.771) (end 115.108 74.275) (width 0.25) (layer B.Cu) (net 21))
 (segment (start 155.24 75.545) (end 155.24 79.355) (width 0.254) (layer F.Cu) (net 22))
 (segment (start 155.24 69.195) (end 155.24 73.005) (width 0.254) (layer F.Cu) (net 23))
 (segment (start 155.24 62.845) (end 155.24 66.655) (width 0.254) (layer F.Cu) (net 24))
 (segment (start 112.903 75.946) (end 113.236 75.946) (width 0.25) (layer B.Cu) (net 25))
 (segment (start 105.41 75.946) (end 112.903 75.946) (width 0.254) (layer B.Cu) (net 25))
 (segment (start 113.236 75.946) (end 114.359 77.069) (width 0.25) (layer B.Cu) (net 25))
 (segment (start 114.346 77.069) (end 114.359 77.069) (width 0.254) (layer B.Cu) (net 25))
 (segment (start 114.359 77.069) (end 150.922 77.069) (width 0.254) (layer B.Cu) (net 25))
 (via (at 150.922 77.069) (size 0.6) (drill 0.4) (layers F.Cu B.Cu) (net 25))
 (segment (start 150.922 77.069) (end 152.319 75.672) (width 0.254) (layer F.Cu) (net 25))
 (segment (start 152.319 75.672) (end 152.319 63.226) (width 0.254) (layer F.Cu) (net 25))
 (segment (start 155.24 60.305) (end 152.319 63.226) (width 0.254) (layer F.Cu) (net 25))
 (segment (start 162.225 75.545) (end 162.225 79.355) (width 0.254) (layer F.Cu) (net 26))
 (segment (start 162.225 69.195) (end 162.225 73.005) (width 0.254) (layer F.Cu) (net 27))
 (segment (start 162.225 62.845) (end 162.225 66.655) (width 0.254) (layer F.Cu) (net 28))
 (segment (start 113 79.121) (end 113.31 79.121) (width 0.25) (layer B.Cu) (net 29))
 (segment (start 158.923 63.607) (end 162.225 60.305) (width 0.254) (layer F.Cu) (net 29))
 (segment (start 158.923 76.815) (end 158.923 63.607) (width 0.254) (layer F.Cu) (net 29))
 (segment (start 158.034 77.704) (end 158.923 76.815) (width 0.254) (layer F.Cu) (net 29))
 (via (at 158.034 77.704) (size 0.6) (drill 0.4) (layers F.Cu B.Cu) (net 29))
 (segment (start 114.727 77.704) (end 158.034 77.704) (width 0.254) (layer B.Cu) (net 29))
 (segment (start 113.31 79.121) (end 114.727 77.704) (width 0.25) (layer B.Cu) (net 29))
 (segment (start 105.41 79.121) (end 113 79.121) (width 0.254) (layer B.Cu) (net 29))
 (segment (start 113 79.121) (end 113.03 79.121) (width 0.254) (layer B.Cu) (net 29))
 (segment (start 169.21 75.545) (end 169.21 79.355) (width 0.254) (layer F.Cu) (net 30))
 (segment (start 169.21 69.195) (end 169.21 73.005) (width 0.254) (layer F.Cu) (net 31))
 (segment (start 169.21 62.845) (end 169.21 66.655) (width 0.254) (layer F.Cu) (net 32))
 (segment (start 112.395 82.296) (end 112.675 82.296) (width 0.25) (layer B.Cu) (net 33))
 (segment (start 105.41 82.296) (end 112.395 82.296) (width 0.254) (layer B.Cu) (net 33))
 (segment (start 166.67 62.845) (end 169.21 60.305) (width 0.254) (layer F.Cu) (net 33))
 (segment (start 166.67 79.101) (end 166.67 62.845) (width 0.254) (layer F.Cu) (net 33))
 (segment (start 165.146 80.625) (end 166.67 79.101) (width 0.254) (layer F.Cu) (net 33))
 (via (at 165.146 80.625) (size 0.6) (drill 0.4) (layers F.Cu B.Cu) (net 33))
 (segment (start 114.346 80.625) (end 165.146 80.625) (width 0.254) (layer B.Cu) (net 33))
 (segment (start 112.675 82.296) (end 114.346 80.625) (width 0.25) (layer B.Cu) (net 33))
 (segment (start 189.23 72.35) (end 174.45 72.35) (width 0.25) (layer B.Cu) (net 34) (status 400000))
 (segment (start 117.65 70.56) (end 115.57 72.64) (width 0.25) (layer F.Cu) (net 34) (status 800000))
 (via (at 117.65 70.56) (size 0.6) (drill 0.4) (layers F.Cu B.Cu) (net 34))
 (segment (start 172.66 70.56) (end 117.65 70.56) (width 0.25) (layer B.Cu) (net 34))
 (segment (start 174.45 72.35) (end 172.66 70.56) (width 0.25) (layer B.Cu) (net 34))
 (segment (start 115.57 72.64) (end 115.57 72.771) (width 0.25) (layer F.Cu) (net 34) (status C00000))
 (segment (start 115.697 72.771) (end 115.57 72.771) (width 0.25) (layer F.Cu) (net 34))
 (segment (start 115.57 63.246) (end 115.57 60.071) (width 0.25) (layer F.Cu) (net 34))
 (segment (start 115.57 66.421) (end 115.57 63.246) (width 0.25) (layer F.Cu) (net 34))
 (segment (start 115.57 69.596) (end 115.57 66.421) (width 0.25) (layer F.Cu) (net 34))
 (segment (start 115.57 72.771) (end 115.57 69.596) (width 0.25) (layer F.Cu) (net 34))
 (segment (start 115.57 75.946) (end 115.57 72.771) (width 0.25) (layer F.Cu) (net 34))
 (segment (start 115.57 79.121) (end 115.57 75.946) (width 0.25) (layer F.Cu) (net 34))
 (segment (start 115.57 82.296) (end 115.57 79.121) (width 0.25) (layer F.Cu) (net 34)))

